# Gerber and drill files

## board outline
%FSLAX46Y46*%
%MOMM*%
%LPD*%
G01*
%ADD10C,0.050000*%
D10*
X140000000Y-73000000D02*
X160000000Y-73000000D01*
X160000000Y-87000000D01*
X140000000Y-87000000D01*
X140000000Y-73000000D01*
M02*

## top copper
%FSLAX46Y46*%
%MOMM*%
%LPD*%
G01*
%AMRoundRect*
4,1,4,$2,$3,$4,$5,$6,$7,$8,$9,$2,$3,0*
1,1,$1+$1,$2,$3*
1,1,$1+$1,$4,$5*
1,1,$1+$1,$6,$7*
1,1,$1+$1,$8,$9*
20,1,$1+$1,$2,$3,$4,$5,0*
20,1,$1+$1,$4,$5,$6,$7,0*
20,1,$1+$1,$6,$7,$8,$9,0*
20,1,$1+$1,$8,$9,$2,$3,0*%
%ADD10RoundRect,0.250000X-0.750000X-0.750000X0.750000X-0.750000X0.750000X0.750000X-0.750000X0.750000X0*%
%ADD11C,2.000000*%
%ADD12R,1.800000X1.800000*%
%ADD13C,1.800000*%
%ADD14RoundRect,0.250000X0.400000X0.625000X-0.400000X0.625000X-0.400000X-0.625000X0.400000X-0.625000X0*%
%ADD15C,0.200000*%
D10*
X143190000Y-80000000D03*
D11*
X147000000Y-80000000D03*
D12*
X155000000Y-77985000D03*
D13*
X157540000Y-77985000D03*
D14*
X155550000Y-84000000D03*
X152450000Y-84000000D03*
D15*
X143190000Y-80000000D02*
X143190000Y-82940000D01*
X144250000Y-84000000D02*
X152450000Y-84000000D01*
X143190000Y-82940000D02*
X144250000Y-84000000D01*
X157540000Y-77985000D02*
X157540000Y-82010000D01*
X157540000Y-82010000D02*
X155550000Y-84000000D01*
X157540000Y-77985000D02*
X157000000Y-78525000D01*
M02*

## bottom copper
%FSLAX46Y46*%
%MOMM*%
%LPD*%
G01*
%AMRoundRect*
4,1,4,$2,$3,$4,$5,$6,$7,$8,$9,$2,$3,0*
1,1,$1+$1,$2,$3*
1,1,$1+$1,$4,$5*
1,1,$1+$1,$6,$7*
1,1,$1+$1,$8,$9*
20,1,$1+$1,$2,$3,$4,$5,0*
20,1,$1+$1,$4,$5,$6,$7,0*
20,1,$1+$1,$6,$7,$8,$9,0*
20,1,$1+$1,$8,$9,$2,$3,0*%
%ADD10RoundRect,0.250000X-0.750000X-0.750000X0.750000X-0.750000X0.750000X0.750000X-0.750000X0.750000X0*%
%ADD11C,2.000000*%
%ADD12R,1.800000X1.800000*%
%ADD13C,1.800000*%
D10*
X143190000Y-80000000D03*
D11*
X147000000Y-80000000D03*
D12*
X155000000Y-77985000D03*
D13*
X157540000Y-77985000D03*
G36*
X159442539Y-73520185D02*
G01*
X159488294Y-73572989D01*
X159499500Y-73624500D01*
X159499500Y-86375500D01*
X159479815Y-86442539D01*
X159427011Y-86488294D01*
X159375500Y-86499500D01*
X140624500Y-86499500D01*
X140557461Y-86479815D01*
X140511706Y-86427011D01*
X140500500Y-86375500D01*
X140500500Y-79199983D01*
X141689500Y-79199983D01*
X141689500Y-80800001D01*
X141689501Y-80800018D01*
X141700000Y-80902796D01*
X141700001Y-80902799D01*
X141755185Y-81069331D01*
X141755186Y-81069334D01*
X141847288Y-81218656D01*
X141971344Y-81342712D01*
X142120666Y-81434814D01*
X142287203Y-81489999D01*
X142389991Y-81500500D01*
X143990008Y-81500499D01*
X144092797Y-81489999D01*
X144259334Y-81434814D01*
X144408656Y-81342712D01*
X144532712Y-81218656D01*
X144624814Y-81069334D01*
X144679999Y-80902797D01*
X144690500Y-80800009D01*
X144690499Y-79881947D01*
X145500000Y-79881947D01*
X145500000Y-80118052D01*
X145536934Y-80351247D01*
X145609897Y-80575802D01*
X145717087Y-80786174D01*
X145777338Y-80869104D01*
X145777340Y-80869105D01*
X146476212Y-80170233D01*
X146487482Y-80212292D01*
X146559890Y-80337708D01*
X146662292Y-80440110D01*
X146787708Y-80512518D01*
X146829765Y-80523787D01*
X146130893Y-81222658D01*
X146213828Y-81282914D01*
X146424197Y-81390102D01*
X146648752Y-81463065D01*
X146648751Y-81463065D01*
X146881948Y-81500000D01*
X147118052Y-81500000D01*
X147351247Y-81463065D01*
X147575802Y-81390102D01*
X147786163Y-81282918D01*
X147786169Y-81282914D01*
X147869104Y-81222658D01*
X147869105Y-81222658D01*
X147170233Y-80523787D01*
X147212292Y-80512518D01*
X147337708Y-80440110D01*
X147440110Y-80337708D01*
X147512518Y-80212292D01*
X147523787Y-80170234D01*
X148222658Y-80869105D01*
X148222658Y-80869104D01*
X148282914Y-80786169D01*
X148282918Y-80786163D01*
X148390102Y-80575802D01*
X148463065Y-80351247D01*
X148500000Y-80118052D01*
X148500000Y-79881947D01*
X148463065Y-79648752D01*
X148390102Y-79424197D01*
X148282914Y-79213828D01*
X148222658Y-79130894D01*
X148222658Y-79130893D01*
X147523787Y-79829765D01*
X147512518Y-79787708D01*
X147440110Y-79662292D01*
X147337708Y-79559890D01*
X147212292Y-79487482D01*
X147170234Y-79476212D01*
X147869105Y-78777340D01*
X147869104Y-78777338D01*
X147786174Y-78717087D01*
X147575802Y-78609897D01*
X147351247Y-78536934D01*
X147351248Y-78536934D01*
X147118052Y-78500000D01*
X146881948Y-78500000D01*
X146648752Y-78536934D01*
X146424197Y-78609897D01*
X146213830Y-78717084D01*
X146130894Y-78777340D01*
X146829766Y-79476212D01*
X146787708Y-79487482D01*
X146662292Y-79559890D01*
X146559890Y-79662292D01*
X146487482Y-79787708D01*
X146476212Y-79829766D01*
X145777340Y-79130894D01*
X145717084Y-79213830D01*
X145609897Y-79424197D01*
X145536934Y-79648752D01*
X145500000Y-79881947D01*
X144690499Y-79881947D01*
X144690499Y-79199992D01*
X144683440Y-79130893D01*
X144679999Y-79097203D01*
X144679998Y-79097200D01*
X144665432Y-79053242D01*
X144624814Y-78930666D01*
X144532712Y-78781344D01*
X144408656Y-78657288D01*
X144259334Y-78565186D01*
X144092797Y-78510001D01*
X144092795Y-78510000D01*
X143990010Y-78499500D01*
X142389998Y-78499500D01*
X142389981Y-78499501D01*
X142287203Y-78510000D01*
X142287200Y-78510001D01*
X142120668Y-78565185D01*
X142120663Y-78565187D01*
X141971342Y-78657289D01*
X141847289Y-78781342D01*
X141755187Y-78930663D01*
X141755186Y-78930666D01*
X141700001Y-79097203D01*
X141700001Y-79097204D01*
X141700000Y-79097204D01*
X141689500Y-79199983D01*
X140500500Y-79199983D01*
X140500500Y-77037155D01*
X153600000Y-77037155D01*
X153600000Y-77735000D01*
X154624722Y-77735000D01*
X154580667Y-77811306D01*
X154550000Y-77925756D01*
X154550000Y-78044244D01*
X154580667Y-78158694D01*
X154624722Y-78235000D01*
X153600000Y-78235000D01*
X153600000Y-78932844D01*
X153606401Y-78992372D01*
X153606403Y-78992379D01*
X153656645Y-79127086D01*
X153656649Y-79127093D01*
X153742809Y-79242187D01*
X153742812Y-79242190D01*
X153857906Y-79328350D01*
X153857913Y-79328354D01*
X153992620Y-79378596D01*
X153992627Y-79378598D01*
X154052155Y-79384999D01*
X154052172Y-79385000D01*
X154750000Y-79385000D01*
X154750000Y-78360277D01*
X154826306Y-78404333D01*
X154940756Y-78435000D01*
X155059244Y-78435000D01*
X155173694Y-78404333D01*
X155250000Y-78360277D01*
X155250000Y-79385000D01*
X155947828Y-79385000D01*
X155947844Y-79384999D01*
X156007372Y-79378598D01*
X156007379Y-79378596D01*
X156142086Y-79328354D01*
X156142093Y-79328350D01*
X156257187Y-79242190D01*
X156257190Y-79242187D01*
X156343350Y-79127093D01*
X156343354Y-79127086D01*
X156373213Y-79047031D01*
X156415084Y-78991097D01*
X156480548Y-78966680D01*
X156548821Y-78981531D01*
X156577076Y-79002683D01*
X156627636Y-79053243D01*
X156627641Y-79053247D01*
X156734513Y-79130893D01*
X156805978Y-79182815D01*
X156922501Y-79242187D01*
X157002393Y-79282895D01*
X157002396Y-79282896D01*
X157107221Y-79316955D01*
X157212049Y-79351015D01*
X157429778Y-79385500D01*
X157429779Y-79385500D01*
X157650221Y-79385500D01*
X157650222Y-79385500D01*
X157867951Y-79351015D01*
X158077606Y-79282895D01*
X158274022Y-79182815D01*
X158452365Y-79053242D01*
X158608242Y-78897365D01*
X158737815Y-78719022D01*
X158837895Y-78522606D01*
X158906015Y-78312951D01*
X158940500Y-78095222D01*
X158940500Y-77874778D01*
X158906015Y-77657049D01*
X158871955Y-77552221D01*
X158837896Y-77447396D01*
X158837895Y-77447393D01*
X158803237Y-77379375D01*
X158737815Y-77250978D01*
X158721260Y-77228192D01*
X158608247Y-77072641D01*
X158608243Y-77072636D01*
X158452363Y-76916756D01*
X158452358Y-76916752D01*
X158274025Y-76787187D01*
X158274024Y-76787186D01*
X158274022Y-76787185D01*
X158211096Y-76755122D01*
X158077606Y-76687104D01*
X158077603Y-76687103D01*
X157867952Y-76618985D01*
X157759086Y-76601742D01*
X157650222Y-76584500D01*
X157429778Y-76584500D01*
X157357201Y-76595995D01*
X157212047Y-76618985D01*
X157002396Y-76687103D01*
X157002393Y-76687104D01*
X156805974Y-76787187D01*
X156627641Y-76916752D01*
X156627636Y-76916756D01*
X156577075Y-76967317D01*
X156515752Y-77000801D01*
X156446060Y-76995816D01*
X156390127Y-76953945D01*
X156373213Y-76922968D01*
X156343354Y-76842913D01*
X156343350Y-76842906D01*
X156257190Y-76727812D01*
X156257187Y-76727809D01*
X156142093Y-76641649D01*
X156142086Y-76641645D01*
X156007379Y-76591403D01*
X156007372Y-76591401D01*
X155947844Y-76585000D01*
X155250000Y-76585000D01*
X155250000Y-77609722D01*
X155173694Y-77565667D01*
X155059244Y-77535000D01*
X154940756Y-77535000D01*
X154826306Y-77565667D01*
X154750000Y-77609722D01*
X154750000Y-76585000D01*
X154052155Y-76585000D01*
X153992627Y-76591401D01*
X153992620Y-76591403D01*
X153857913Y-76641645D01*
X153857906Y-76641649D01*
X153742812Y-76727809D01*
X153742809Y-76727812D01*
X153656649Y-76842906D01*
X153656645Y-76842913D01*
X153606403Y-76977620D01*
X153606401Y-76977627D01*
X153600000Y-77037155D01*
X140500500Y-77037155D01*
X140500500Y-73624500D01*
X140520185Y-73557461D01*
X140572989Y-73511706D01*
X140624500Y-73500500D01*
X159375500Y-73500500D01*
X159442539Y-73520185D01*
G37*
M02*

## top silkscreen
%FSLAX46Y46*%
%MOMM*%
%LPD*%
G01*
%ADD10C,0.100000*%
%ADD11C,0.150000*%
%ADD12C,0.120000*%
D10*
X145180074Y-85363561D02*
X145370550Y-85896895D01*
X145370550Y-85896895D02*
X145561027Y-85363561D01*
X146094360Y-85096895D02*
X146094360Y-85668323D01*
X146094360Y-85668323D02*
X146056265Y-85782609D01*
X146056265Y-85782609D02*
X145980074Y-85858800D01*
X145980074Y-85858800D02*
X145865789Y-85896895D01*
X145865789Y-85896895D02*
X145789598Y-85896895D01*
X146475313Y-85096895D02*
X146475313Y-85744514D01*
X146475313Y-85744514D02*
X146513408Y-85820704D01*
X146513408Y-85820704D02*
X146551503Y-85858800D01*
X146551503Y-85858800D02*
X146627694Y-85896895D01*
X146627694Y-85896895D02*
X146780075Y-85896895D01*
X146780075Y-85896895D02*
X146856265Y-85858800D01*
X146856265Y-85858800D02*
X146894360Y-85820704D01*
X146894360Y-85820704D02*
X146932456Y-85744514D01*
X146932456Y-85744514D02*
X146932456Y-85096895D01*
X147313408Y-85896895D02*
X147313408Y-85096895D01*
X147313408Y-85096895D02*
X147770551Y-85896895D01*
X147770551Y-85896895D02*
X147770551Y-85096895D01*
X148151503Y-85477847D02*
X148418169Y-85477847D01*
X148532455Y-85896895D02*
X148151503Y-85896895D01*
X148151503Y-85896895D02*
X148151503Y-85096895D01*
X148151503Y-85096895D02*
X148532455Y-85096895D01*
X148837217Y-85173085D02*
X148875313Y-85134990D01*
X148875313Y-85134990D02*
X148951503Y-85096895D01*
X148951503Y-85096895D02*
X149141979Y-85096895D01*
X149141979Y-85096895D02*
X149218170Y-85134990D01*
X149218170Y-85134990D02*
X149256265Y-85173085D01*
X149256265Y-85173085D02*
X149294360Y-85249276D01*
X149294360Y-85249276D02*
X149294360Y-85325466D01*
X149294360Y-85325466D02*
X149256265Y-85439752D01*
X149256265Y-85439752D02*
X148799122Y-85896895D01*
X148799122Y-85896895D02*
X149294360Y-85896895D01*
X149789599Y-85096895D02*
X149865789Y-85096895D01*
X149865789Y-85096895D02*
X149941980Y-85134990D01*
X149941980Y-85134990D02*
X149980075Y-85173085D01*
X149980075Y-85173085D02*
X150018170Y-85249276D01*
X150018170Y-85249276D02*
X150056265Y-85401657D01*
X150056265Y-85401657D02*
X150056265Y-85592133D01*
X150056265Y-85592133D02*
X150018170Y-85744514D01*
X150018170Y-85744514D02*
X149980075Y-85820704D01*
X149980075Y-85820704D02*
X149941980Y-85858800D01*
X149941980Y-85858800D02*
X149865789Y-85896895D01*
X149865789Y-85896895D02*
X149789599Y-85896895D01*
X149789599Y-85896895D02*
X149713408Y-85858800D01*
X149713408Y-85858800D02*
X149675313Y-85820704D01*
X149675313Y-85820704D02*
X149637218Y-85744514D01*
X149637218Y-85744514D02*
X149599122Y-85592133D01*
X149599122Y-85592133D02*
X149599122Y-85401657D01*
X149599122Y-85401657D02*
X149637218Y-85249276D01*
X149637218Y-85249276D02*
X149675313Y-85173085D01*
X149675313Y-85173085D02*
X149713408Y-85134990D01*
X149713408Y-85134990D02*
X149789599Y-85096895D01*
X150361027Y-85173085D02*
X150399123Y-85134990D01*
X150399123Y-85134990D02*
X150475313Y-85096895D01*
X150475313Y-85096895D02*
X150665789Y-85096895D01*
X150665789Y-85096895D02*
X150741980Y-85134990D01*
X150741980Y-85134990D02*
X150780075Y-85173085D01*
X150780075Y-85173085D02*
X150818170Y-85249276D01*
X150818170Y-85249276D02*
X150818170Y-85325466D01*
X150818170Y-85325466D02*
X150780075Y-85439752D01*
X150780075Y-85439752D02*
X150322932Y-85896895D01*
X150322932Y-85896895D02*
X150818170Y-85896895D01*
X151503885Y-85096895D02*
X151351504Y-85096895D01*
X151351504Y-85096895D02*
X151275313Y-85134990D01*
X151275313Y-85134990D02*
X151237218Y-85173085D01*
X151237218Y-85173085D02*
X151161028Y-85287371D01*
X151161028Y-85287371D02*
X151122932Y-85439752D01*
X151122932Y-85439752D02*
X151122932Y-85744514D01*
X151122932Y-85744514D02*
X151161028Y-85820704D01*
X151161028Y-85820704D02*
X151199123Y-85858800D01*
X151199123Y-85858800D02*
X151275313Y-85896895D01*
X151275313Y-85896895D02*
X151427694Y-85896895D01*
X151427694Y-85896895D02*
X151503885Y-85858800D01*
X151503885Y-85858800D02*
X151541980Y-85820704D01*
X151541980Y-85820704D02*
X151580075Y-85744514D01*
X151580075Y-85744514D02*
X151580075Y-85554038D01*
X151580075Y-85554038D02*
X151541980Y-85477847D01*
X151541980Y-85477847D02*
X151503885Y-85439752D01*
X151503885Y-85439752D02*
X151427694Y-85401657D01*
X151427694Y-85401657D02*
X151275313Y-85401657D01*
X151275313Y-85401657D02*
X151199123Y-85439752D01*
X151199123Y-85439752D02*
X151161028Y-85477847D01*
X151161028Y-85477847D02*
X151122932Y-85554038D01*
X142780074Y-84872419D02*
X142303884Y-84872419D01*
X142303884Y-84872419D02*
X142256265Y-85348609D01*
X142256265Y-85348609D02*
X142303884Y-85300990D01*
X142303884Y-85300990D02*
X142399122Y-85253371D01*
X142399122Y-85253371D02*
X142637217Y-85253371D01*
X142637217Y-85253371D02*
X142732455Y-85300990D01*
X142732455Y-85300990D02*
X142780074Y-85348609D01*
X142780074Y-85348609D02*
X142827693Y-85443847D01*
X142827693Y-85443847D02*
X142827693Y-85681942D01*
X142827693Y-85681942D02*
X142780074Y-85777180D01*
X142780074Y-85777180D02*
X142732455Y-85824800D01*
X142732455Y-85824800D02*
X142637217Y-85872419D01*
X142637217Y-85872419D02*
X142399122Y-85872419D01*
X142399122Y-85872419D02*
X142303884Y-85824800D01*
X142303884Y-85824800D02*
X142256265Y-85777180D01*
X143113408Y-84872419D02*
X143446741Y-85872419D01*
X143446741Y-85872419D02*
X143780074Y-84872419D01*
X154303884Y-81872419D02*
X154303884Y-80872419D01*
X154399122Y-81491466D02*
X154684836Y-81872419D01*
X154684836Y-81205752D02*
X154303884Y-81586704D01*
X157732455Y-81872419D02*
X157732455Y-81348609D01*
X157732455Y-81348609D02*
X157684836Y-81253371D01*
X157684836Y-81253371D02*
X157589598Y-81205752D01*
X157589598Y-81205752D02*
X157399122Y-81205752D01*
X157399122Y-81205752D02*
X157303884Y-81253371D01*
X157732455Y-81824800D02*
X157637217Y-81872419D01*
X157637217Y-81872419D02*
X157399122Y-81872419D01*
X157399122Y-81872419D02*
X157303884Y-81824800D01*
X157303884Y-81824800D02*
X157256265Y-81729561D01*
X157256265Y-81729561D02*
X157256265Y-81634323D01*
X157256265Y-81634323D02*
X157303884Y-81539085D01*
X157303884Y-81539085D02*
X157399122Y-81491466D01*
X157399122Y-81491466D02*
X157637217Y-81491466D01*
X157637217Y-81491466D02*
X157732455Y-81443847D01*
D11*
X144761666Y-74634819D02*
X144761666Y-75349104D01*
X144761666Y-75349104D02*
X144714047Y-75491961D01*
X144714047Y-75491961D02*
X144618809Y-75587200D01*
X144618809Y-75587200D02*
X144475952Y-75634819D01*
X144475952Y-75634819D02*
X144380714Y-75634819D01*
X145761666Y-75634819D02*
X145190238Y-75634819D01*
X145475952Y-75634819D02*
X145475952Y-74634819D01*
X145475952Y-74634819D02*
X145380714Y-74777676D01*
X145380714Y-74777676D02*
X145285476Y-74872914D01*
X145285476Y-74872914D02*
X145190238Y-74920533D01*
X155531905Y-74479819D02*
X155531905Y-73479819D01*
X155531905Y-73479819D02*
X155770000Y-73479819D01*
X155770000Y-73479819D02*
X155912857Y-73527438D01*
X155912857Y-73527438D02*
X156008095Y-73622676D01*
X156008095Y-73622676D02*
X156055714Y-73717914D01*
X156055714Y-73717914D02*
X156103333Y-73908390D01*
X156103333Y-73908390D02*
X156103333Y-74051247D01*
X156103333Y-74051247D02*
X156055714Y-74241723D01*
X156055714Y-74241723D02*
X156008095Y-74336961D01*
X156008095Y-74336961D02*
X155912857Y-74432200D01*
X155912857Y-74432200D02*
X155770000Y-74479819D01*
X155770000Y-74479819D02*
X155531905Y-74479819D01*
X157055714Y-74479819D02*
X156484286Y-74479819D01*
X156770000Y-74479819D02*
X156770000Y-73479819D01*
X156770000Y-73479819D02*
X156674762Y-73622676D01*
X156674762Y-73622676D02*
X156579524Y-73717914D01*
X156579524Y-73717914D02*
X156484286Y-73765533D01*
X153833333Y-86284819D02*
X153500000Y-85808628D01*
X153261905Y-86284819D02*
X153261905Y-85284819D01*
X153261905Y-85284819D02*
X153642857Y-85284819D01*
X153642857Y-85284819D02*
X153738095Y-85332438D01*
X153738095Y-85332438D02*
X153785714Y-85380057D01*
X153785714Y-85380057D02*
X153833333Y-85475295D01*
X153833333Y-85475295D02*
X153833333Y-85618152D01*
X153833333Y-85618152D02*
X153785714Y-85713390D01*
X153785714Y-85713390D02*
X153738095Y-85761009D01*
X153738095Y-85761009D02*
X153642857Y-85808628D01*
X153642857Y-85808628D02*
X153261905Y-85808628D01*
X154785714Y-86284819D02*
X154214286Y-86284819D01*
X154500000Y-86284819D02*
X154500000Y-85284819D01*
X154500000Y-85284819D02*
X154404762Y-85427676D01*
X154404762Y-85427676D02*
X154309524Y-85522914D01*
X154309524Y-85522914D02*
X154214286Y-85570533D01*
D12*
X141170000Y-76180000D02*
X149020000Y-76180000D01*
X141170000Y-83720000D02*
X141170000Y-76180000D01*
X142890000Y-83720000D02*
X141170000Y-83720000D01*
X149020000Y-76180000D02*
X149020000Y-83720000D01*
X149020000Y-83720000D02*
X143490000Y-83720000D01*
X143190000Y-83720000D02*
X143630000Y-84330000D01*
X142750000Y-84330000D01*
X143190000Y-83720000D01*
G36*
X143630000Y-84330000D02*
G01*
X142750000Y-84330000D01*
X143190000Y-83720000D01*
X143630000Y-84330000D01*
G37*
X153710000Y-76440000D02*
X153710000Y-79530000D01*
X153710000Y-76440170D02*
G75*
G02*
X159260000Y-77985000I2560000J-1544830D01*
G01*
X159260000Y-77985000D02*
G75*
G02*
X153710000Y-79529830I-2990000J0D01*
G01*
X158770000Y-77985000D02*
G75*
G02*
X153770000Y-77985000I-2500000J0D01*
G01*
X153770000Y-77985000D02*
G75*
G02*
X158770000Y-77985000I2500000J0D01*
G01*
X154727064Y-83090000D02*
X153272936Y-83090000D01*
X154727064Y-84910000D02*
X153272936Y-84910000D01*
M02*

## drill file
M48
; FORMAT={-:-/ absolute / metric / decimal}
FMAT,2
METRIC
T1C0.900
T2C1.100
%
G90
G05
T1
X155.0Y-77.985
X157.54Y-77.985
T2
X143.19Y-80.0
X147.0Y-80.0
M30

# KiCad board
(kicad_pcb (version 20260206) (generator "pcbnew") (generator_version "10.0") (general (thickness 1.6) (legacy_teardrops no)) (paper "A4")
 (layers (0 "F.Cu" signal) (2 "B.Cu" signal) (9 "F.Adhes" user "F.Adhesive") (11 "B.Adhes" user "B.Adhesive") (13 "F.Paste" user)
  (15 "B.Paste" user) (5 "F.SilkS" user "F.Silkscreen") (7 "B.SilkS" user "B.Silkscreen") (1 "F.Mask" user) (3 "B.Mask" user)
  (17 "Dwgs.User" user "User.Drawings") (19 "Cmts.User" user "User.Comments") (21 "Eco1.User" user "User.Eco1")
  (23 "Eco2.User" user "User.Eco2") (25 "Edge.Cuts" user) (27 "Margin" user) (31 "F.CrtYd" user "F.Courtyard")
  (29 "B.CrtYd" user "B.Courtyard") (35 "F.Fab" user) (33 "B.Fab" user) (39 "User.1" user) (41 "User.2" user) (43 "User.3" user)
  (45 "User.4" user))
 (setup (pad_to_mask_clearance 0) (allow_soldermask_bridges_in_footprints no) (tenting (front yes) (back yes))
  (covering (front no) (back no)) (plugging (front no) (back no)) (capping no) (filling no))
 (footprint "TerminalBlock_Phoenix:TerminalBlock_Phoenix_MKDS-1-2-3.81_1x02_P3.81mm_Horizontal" (layer "F.Cu") (at 143.19 80)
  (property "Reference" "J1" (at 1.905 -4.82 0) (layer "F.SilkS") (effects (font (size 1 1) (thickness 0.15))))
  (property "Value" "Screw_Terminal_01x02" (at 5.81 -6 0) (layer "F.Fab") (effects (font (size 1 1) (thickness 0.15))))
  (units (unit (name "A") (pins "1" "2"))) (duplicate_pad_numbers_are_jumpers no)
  (fp_line (start -2.02 -3.82) (end 5.83 -3.82) (stroke (width 0.12) (type solid)) (layer "F.SilkS"))
  (fp_line (start -2.02 3.72) (end -2.02 -3.82) (stroke (width 0.12) (type solid)) (layer "F.SilkS"))
  (fp_line (start -0.3 3.72) (end -2.02 3.72) (stroke (width 0.12) (type solid)) (layer "F.SilkS"))
  (fp_line (start 5.83 -3.82) (end 5.83 3.72) (stroke (width 0.12) (type solid)) (layer "F.SilkS"))
  (fp_line (start 5.83 3.72) (end 0.3 3.72) (stroke (width 0.12) (type solid)) (layer "F.SilkS"))
  (fp_poly (pts (xy 0 3.72) (xy 0.44 4.33) (xy -0.44 4.33)) (stroke (width 0.12) (type solid)) (fill yes) (layer "F.SilkS"))
  (pad "1" thru_hole roundrect (at 0 0) (size 2 2) (drill 1.1) (layers "*.Cu" "*.Mask") (remove_unused_layers no) (roundrect_rratio 0.125)
   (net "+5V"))
  (pad "2" thru_hole circle (at 3.81 0) (size 2 2) (drill 1.1) (layers "*.Cu" "*.Mask") (remove_unused_layers no) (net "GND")))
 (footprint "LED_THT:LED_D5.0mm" (layer "F.Cu") (at 155 77.985)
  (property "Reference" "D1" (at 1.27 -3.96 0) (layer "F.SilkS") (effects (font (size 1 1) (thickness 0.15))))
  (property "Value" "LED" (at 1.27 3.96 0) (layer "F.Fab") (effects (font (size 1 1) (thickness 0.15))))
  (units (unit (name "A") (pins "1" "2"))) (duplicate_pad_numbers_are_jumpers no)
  (fp_line (start -1.29 -1.545) (end -1.29 1.545) (stroke (width 0.12) (type solid)) (layer "F.SilkS"))
  (fp_arc (start -1.29 -1.54483) (mid 2.071779 -2.880495) (end 4.26 0) (stroke (width 0.12) (type solid)) (layer "F.SilkS"))
  (fp_arc (start 4.26 0) (mid 2.071779 2.880495) (end -1.29 1.54483) (stroke (width 0.12) (type solid)) (layer "F.SilkS"))
  (fp_circle (center 1.27 0) (end 3.77 0) (stroke (width 0.12) (type solid)) (fill no) (layer "F.SilkS"))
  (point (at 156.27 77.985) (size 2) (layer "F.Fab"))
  (pad "1" thru_hole rect (at 0 0) (size 1.8 1.8) (drill 0.9) (layers "*.Cu" "*.Mask") (remove_unused_layers no) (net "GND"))
  (pad "2" thru_hole circle (at 2.54 0) (size 1.8 1.8) (drill 0.9) (layers "*.Cu" "*.Mask") (remove_unused_layers no) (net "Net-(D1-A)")))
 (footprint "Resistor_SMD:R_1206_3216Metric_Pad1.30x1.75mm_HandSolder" (layer "F.Cu") (at 154 84 180)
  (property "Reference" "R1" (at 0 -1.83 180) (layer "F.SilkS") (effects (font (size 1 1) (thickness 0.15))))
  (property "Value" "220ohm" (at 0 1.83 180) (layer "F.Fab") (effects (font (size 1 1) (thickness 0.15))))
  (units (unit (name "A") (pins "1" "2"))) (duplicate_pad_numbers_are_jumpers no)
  (fp_line (start -0.727064 0.91) (end 0.727064 0.91) (stroke (width 0.12) (type solid)) (layer "F.SilkS"))
  (fp_line (start -0.727064 -0.91) (end 0.727064 -0.91) (stroke (width 0.12) (type solid)) (layer "F.SilkS"))
  (pad "1" smd roundrect (at -1.55 0 180) (size 1.3 1.75) (layers "F.Cu" "F.Mask" "F.Paste") (roundrect_rratio 0.192308) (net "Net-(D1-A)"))
  (pad "2" smd roundrect (at 1.55 0 180) (size 1.3 1.75) (layers "F.Cu" "F.Mask" "F.Paste") (roundrect_rratio 0.192308) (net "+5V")))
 (gr_rect (start 140 73) (end 160 87) (stroke (width 0.05) (type default)) (fill no) (layer "Edge.Cuts"))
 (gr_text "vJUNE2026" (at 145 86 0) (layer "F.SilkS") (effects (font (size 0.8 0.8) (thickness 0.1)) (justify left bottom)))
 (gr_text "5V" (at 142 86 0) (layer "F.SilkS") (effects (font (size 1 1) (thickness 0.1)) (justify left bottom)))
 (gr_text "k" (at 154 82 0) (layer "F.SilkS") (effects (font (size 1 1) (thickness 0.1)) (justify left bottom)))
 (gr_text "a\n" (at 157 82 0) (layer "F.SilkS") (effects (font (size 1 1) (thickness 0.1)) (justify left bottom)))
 (segment (start 143.19 80) (end 143.19 82.94) (width 0.2) (layer "F.Cu") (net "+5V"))
 (segment (start 144.25 84) (end 152.45 84) (width 0.2) (layer "F.Cu") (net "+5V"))
 (segment (start 143.19 82.94) (end 144.25 84) (width 0.2) (layer "F.Cu") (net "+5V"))
 (segment (start 157.54 77.985) (end 157.54 82.01) (width 0.2) (layer "F.Cu") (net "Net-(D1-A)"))
 (segment (start 157.54 82.01) (end 155.55 84) (width 0.2) (layer "F.Cu") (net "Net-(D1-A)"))
 (segment (start 157.54 77.985) (end 157 78.525) (width 0.2) (layer "F.Cu") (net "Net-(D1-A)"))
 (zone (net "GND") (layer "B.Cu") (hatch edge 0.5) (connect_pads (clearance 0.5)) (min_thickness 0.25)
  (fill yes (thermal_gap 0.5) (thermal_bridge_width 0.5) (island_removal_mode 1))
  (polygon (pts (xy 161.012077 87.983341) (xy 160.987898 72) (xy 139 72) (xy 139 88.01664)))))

